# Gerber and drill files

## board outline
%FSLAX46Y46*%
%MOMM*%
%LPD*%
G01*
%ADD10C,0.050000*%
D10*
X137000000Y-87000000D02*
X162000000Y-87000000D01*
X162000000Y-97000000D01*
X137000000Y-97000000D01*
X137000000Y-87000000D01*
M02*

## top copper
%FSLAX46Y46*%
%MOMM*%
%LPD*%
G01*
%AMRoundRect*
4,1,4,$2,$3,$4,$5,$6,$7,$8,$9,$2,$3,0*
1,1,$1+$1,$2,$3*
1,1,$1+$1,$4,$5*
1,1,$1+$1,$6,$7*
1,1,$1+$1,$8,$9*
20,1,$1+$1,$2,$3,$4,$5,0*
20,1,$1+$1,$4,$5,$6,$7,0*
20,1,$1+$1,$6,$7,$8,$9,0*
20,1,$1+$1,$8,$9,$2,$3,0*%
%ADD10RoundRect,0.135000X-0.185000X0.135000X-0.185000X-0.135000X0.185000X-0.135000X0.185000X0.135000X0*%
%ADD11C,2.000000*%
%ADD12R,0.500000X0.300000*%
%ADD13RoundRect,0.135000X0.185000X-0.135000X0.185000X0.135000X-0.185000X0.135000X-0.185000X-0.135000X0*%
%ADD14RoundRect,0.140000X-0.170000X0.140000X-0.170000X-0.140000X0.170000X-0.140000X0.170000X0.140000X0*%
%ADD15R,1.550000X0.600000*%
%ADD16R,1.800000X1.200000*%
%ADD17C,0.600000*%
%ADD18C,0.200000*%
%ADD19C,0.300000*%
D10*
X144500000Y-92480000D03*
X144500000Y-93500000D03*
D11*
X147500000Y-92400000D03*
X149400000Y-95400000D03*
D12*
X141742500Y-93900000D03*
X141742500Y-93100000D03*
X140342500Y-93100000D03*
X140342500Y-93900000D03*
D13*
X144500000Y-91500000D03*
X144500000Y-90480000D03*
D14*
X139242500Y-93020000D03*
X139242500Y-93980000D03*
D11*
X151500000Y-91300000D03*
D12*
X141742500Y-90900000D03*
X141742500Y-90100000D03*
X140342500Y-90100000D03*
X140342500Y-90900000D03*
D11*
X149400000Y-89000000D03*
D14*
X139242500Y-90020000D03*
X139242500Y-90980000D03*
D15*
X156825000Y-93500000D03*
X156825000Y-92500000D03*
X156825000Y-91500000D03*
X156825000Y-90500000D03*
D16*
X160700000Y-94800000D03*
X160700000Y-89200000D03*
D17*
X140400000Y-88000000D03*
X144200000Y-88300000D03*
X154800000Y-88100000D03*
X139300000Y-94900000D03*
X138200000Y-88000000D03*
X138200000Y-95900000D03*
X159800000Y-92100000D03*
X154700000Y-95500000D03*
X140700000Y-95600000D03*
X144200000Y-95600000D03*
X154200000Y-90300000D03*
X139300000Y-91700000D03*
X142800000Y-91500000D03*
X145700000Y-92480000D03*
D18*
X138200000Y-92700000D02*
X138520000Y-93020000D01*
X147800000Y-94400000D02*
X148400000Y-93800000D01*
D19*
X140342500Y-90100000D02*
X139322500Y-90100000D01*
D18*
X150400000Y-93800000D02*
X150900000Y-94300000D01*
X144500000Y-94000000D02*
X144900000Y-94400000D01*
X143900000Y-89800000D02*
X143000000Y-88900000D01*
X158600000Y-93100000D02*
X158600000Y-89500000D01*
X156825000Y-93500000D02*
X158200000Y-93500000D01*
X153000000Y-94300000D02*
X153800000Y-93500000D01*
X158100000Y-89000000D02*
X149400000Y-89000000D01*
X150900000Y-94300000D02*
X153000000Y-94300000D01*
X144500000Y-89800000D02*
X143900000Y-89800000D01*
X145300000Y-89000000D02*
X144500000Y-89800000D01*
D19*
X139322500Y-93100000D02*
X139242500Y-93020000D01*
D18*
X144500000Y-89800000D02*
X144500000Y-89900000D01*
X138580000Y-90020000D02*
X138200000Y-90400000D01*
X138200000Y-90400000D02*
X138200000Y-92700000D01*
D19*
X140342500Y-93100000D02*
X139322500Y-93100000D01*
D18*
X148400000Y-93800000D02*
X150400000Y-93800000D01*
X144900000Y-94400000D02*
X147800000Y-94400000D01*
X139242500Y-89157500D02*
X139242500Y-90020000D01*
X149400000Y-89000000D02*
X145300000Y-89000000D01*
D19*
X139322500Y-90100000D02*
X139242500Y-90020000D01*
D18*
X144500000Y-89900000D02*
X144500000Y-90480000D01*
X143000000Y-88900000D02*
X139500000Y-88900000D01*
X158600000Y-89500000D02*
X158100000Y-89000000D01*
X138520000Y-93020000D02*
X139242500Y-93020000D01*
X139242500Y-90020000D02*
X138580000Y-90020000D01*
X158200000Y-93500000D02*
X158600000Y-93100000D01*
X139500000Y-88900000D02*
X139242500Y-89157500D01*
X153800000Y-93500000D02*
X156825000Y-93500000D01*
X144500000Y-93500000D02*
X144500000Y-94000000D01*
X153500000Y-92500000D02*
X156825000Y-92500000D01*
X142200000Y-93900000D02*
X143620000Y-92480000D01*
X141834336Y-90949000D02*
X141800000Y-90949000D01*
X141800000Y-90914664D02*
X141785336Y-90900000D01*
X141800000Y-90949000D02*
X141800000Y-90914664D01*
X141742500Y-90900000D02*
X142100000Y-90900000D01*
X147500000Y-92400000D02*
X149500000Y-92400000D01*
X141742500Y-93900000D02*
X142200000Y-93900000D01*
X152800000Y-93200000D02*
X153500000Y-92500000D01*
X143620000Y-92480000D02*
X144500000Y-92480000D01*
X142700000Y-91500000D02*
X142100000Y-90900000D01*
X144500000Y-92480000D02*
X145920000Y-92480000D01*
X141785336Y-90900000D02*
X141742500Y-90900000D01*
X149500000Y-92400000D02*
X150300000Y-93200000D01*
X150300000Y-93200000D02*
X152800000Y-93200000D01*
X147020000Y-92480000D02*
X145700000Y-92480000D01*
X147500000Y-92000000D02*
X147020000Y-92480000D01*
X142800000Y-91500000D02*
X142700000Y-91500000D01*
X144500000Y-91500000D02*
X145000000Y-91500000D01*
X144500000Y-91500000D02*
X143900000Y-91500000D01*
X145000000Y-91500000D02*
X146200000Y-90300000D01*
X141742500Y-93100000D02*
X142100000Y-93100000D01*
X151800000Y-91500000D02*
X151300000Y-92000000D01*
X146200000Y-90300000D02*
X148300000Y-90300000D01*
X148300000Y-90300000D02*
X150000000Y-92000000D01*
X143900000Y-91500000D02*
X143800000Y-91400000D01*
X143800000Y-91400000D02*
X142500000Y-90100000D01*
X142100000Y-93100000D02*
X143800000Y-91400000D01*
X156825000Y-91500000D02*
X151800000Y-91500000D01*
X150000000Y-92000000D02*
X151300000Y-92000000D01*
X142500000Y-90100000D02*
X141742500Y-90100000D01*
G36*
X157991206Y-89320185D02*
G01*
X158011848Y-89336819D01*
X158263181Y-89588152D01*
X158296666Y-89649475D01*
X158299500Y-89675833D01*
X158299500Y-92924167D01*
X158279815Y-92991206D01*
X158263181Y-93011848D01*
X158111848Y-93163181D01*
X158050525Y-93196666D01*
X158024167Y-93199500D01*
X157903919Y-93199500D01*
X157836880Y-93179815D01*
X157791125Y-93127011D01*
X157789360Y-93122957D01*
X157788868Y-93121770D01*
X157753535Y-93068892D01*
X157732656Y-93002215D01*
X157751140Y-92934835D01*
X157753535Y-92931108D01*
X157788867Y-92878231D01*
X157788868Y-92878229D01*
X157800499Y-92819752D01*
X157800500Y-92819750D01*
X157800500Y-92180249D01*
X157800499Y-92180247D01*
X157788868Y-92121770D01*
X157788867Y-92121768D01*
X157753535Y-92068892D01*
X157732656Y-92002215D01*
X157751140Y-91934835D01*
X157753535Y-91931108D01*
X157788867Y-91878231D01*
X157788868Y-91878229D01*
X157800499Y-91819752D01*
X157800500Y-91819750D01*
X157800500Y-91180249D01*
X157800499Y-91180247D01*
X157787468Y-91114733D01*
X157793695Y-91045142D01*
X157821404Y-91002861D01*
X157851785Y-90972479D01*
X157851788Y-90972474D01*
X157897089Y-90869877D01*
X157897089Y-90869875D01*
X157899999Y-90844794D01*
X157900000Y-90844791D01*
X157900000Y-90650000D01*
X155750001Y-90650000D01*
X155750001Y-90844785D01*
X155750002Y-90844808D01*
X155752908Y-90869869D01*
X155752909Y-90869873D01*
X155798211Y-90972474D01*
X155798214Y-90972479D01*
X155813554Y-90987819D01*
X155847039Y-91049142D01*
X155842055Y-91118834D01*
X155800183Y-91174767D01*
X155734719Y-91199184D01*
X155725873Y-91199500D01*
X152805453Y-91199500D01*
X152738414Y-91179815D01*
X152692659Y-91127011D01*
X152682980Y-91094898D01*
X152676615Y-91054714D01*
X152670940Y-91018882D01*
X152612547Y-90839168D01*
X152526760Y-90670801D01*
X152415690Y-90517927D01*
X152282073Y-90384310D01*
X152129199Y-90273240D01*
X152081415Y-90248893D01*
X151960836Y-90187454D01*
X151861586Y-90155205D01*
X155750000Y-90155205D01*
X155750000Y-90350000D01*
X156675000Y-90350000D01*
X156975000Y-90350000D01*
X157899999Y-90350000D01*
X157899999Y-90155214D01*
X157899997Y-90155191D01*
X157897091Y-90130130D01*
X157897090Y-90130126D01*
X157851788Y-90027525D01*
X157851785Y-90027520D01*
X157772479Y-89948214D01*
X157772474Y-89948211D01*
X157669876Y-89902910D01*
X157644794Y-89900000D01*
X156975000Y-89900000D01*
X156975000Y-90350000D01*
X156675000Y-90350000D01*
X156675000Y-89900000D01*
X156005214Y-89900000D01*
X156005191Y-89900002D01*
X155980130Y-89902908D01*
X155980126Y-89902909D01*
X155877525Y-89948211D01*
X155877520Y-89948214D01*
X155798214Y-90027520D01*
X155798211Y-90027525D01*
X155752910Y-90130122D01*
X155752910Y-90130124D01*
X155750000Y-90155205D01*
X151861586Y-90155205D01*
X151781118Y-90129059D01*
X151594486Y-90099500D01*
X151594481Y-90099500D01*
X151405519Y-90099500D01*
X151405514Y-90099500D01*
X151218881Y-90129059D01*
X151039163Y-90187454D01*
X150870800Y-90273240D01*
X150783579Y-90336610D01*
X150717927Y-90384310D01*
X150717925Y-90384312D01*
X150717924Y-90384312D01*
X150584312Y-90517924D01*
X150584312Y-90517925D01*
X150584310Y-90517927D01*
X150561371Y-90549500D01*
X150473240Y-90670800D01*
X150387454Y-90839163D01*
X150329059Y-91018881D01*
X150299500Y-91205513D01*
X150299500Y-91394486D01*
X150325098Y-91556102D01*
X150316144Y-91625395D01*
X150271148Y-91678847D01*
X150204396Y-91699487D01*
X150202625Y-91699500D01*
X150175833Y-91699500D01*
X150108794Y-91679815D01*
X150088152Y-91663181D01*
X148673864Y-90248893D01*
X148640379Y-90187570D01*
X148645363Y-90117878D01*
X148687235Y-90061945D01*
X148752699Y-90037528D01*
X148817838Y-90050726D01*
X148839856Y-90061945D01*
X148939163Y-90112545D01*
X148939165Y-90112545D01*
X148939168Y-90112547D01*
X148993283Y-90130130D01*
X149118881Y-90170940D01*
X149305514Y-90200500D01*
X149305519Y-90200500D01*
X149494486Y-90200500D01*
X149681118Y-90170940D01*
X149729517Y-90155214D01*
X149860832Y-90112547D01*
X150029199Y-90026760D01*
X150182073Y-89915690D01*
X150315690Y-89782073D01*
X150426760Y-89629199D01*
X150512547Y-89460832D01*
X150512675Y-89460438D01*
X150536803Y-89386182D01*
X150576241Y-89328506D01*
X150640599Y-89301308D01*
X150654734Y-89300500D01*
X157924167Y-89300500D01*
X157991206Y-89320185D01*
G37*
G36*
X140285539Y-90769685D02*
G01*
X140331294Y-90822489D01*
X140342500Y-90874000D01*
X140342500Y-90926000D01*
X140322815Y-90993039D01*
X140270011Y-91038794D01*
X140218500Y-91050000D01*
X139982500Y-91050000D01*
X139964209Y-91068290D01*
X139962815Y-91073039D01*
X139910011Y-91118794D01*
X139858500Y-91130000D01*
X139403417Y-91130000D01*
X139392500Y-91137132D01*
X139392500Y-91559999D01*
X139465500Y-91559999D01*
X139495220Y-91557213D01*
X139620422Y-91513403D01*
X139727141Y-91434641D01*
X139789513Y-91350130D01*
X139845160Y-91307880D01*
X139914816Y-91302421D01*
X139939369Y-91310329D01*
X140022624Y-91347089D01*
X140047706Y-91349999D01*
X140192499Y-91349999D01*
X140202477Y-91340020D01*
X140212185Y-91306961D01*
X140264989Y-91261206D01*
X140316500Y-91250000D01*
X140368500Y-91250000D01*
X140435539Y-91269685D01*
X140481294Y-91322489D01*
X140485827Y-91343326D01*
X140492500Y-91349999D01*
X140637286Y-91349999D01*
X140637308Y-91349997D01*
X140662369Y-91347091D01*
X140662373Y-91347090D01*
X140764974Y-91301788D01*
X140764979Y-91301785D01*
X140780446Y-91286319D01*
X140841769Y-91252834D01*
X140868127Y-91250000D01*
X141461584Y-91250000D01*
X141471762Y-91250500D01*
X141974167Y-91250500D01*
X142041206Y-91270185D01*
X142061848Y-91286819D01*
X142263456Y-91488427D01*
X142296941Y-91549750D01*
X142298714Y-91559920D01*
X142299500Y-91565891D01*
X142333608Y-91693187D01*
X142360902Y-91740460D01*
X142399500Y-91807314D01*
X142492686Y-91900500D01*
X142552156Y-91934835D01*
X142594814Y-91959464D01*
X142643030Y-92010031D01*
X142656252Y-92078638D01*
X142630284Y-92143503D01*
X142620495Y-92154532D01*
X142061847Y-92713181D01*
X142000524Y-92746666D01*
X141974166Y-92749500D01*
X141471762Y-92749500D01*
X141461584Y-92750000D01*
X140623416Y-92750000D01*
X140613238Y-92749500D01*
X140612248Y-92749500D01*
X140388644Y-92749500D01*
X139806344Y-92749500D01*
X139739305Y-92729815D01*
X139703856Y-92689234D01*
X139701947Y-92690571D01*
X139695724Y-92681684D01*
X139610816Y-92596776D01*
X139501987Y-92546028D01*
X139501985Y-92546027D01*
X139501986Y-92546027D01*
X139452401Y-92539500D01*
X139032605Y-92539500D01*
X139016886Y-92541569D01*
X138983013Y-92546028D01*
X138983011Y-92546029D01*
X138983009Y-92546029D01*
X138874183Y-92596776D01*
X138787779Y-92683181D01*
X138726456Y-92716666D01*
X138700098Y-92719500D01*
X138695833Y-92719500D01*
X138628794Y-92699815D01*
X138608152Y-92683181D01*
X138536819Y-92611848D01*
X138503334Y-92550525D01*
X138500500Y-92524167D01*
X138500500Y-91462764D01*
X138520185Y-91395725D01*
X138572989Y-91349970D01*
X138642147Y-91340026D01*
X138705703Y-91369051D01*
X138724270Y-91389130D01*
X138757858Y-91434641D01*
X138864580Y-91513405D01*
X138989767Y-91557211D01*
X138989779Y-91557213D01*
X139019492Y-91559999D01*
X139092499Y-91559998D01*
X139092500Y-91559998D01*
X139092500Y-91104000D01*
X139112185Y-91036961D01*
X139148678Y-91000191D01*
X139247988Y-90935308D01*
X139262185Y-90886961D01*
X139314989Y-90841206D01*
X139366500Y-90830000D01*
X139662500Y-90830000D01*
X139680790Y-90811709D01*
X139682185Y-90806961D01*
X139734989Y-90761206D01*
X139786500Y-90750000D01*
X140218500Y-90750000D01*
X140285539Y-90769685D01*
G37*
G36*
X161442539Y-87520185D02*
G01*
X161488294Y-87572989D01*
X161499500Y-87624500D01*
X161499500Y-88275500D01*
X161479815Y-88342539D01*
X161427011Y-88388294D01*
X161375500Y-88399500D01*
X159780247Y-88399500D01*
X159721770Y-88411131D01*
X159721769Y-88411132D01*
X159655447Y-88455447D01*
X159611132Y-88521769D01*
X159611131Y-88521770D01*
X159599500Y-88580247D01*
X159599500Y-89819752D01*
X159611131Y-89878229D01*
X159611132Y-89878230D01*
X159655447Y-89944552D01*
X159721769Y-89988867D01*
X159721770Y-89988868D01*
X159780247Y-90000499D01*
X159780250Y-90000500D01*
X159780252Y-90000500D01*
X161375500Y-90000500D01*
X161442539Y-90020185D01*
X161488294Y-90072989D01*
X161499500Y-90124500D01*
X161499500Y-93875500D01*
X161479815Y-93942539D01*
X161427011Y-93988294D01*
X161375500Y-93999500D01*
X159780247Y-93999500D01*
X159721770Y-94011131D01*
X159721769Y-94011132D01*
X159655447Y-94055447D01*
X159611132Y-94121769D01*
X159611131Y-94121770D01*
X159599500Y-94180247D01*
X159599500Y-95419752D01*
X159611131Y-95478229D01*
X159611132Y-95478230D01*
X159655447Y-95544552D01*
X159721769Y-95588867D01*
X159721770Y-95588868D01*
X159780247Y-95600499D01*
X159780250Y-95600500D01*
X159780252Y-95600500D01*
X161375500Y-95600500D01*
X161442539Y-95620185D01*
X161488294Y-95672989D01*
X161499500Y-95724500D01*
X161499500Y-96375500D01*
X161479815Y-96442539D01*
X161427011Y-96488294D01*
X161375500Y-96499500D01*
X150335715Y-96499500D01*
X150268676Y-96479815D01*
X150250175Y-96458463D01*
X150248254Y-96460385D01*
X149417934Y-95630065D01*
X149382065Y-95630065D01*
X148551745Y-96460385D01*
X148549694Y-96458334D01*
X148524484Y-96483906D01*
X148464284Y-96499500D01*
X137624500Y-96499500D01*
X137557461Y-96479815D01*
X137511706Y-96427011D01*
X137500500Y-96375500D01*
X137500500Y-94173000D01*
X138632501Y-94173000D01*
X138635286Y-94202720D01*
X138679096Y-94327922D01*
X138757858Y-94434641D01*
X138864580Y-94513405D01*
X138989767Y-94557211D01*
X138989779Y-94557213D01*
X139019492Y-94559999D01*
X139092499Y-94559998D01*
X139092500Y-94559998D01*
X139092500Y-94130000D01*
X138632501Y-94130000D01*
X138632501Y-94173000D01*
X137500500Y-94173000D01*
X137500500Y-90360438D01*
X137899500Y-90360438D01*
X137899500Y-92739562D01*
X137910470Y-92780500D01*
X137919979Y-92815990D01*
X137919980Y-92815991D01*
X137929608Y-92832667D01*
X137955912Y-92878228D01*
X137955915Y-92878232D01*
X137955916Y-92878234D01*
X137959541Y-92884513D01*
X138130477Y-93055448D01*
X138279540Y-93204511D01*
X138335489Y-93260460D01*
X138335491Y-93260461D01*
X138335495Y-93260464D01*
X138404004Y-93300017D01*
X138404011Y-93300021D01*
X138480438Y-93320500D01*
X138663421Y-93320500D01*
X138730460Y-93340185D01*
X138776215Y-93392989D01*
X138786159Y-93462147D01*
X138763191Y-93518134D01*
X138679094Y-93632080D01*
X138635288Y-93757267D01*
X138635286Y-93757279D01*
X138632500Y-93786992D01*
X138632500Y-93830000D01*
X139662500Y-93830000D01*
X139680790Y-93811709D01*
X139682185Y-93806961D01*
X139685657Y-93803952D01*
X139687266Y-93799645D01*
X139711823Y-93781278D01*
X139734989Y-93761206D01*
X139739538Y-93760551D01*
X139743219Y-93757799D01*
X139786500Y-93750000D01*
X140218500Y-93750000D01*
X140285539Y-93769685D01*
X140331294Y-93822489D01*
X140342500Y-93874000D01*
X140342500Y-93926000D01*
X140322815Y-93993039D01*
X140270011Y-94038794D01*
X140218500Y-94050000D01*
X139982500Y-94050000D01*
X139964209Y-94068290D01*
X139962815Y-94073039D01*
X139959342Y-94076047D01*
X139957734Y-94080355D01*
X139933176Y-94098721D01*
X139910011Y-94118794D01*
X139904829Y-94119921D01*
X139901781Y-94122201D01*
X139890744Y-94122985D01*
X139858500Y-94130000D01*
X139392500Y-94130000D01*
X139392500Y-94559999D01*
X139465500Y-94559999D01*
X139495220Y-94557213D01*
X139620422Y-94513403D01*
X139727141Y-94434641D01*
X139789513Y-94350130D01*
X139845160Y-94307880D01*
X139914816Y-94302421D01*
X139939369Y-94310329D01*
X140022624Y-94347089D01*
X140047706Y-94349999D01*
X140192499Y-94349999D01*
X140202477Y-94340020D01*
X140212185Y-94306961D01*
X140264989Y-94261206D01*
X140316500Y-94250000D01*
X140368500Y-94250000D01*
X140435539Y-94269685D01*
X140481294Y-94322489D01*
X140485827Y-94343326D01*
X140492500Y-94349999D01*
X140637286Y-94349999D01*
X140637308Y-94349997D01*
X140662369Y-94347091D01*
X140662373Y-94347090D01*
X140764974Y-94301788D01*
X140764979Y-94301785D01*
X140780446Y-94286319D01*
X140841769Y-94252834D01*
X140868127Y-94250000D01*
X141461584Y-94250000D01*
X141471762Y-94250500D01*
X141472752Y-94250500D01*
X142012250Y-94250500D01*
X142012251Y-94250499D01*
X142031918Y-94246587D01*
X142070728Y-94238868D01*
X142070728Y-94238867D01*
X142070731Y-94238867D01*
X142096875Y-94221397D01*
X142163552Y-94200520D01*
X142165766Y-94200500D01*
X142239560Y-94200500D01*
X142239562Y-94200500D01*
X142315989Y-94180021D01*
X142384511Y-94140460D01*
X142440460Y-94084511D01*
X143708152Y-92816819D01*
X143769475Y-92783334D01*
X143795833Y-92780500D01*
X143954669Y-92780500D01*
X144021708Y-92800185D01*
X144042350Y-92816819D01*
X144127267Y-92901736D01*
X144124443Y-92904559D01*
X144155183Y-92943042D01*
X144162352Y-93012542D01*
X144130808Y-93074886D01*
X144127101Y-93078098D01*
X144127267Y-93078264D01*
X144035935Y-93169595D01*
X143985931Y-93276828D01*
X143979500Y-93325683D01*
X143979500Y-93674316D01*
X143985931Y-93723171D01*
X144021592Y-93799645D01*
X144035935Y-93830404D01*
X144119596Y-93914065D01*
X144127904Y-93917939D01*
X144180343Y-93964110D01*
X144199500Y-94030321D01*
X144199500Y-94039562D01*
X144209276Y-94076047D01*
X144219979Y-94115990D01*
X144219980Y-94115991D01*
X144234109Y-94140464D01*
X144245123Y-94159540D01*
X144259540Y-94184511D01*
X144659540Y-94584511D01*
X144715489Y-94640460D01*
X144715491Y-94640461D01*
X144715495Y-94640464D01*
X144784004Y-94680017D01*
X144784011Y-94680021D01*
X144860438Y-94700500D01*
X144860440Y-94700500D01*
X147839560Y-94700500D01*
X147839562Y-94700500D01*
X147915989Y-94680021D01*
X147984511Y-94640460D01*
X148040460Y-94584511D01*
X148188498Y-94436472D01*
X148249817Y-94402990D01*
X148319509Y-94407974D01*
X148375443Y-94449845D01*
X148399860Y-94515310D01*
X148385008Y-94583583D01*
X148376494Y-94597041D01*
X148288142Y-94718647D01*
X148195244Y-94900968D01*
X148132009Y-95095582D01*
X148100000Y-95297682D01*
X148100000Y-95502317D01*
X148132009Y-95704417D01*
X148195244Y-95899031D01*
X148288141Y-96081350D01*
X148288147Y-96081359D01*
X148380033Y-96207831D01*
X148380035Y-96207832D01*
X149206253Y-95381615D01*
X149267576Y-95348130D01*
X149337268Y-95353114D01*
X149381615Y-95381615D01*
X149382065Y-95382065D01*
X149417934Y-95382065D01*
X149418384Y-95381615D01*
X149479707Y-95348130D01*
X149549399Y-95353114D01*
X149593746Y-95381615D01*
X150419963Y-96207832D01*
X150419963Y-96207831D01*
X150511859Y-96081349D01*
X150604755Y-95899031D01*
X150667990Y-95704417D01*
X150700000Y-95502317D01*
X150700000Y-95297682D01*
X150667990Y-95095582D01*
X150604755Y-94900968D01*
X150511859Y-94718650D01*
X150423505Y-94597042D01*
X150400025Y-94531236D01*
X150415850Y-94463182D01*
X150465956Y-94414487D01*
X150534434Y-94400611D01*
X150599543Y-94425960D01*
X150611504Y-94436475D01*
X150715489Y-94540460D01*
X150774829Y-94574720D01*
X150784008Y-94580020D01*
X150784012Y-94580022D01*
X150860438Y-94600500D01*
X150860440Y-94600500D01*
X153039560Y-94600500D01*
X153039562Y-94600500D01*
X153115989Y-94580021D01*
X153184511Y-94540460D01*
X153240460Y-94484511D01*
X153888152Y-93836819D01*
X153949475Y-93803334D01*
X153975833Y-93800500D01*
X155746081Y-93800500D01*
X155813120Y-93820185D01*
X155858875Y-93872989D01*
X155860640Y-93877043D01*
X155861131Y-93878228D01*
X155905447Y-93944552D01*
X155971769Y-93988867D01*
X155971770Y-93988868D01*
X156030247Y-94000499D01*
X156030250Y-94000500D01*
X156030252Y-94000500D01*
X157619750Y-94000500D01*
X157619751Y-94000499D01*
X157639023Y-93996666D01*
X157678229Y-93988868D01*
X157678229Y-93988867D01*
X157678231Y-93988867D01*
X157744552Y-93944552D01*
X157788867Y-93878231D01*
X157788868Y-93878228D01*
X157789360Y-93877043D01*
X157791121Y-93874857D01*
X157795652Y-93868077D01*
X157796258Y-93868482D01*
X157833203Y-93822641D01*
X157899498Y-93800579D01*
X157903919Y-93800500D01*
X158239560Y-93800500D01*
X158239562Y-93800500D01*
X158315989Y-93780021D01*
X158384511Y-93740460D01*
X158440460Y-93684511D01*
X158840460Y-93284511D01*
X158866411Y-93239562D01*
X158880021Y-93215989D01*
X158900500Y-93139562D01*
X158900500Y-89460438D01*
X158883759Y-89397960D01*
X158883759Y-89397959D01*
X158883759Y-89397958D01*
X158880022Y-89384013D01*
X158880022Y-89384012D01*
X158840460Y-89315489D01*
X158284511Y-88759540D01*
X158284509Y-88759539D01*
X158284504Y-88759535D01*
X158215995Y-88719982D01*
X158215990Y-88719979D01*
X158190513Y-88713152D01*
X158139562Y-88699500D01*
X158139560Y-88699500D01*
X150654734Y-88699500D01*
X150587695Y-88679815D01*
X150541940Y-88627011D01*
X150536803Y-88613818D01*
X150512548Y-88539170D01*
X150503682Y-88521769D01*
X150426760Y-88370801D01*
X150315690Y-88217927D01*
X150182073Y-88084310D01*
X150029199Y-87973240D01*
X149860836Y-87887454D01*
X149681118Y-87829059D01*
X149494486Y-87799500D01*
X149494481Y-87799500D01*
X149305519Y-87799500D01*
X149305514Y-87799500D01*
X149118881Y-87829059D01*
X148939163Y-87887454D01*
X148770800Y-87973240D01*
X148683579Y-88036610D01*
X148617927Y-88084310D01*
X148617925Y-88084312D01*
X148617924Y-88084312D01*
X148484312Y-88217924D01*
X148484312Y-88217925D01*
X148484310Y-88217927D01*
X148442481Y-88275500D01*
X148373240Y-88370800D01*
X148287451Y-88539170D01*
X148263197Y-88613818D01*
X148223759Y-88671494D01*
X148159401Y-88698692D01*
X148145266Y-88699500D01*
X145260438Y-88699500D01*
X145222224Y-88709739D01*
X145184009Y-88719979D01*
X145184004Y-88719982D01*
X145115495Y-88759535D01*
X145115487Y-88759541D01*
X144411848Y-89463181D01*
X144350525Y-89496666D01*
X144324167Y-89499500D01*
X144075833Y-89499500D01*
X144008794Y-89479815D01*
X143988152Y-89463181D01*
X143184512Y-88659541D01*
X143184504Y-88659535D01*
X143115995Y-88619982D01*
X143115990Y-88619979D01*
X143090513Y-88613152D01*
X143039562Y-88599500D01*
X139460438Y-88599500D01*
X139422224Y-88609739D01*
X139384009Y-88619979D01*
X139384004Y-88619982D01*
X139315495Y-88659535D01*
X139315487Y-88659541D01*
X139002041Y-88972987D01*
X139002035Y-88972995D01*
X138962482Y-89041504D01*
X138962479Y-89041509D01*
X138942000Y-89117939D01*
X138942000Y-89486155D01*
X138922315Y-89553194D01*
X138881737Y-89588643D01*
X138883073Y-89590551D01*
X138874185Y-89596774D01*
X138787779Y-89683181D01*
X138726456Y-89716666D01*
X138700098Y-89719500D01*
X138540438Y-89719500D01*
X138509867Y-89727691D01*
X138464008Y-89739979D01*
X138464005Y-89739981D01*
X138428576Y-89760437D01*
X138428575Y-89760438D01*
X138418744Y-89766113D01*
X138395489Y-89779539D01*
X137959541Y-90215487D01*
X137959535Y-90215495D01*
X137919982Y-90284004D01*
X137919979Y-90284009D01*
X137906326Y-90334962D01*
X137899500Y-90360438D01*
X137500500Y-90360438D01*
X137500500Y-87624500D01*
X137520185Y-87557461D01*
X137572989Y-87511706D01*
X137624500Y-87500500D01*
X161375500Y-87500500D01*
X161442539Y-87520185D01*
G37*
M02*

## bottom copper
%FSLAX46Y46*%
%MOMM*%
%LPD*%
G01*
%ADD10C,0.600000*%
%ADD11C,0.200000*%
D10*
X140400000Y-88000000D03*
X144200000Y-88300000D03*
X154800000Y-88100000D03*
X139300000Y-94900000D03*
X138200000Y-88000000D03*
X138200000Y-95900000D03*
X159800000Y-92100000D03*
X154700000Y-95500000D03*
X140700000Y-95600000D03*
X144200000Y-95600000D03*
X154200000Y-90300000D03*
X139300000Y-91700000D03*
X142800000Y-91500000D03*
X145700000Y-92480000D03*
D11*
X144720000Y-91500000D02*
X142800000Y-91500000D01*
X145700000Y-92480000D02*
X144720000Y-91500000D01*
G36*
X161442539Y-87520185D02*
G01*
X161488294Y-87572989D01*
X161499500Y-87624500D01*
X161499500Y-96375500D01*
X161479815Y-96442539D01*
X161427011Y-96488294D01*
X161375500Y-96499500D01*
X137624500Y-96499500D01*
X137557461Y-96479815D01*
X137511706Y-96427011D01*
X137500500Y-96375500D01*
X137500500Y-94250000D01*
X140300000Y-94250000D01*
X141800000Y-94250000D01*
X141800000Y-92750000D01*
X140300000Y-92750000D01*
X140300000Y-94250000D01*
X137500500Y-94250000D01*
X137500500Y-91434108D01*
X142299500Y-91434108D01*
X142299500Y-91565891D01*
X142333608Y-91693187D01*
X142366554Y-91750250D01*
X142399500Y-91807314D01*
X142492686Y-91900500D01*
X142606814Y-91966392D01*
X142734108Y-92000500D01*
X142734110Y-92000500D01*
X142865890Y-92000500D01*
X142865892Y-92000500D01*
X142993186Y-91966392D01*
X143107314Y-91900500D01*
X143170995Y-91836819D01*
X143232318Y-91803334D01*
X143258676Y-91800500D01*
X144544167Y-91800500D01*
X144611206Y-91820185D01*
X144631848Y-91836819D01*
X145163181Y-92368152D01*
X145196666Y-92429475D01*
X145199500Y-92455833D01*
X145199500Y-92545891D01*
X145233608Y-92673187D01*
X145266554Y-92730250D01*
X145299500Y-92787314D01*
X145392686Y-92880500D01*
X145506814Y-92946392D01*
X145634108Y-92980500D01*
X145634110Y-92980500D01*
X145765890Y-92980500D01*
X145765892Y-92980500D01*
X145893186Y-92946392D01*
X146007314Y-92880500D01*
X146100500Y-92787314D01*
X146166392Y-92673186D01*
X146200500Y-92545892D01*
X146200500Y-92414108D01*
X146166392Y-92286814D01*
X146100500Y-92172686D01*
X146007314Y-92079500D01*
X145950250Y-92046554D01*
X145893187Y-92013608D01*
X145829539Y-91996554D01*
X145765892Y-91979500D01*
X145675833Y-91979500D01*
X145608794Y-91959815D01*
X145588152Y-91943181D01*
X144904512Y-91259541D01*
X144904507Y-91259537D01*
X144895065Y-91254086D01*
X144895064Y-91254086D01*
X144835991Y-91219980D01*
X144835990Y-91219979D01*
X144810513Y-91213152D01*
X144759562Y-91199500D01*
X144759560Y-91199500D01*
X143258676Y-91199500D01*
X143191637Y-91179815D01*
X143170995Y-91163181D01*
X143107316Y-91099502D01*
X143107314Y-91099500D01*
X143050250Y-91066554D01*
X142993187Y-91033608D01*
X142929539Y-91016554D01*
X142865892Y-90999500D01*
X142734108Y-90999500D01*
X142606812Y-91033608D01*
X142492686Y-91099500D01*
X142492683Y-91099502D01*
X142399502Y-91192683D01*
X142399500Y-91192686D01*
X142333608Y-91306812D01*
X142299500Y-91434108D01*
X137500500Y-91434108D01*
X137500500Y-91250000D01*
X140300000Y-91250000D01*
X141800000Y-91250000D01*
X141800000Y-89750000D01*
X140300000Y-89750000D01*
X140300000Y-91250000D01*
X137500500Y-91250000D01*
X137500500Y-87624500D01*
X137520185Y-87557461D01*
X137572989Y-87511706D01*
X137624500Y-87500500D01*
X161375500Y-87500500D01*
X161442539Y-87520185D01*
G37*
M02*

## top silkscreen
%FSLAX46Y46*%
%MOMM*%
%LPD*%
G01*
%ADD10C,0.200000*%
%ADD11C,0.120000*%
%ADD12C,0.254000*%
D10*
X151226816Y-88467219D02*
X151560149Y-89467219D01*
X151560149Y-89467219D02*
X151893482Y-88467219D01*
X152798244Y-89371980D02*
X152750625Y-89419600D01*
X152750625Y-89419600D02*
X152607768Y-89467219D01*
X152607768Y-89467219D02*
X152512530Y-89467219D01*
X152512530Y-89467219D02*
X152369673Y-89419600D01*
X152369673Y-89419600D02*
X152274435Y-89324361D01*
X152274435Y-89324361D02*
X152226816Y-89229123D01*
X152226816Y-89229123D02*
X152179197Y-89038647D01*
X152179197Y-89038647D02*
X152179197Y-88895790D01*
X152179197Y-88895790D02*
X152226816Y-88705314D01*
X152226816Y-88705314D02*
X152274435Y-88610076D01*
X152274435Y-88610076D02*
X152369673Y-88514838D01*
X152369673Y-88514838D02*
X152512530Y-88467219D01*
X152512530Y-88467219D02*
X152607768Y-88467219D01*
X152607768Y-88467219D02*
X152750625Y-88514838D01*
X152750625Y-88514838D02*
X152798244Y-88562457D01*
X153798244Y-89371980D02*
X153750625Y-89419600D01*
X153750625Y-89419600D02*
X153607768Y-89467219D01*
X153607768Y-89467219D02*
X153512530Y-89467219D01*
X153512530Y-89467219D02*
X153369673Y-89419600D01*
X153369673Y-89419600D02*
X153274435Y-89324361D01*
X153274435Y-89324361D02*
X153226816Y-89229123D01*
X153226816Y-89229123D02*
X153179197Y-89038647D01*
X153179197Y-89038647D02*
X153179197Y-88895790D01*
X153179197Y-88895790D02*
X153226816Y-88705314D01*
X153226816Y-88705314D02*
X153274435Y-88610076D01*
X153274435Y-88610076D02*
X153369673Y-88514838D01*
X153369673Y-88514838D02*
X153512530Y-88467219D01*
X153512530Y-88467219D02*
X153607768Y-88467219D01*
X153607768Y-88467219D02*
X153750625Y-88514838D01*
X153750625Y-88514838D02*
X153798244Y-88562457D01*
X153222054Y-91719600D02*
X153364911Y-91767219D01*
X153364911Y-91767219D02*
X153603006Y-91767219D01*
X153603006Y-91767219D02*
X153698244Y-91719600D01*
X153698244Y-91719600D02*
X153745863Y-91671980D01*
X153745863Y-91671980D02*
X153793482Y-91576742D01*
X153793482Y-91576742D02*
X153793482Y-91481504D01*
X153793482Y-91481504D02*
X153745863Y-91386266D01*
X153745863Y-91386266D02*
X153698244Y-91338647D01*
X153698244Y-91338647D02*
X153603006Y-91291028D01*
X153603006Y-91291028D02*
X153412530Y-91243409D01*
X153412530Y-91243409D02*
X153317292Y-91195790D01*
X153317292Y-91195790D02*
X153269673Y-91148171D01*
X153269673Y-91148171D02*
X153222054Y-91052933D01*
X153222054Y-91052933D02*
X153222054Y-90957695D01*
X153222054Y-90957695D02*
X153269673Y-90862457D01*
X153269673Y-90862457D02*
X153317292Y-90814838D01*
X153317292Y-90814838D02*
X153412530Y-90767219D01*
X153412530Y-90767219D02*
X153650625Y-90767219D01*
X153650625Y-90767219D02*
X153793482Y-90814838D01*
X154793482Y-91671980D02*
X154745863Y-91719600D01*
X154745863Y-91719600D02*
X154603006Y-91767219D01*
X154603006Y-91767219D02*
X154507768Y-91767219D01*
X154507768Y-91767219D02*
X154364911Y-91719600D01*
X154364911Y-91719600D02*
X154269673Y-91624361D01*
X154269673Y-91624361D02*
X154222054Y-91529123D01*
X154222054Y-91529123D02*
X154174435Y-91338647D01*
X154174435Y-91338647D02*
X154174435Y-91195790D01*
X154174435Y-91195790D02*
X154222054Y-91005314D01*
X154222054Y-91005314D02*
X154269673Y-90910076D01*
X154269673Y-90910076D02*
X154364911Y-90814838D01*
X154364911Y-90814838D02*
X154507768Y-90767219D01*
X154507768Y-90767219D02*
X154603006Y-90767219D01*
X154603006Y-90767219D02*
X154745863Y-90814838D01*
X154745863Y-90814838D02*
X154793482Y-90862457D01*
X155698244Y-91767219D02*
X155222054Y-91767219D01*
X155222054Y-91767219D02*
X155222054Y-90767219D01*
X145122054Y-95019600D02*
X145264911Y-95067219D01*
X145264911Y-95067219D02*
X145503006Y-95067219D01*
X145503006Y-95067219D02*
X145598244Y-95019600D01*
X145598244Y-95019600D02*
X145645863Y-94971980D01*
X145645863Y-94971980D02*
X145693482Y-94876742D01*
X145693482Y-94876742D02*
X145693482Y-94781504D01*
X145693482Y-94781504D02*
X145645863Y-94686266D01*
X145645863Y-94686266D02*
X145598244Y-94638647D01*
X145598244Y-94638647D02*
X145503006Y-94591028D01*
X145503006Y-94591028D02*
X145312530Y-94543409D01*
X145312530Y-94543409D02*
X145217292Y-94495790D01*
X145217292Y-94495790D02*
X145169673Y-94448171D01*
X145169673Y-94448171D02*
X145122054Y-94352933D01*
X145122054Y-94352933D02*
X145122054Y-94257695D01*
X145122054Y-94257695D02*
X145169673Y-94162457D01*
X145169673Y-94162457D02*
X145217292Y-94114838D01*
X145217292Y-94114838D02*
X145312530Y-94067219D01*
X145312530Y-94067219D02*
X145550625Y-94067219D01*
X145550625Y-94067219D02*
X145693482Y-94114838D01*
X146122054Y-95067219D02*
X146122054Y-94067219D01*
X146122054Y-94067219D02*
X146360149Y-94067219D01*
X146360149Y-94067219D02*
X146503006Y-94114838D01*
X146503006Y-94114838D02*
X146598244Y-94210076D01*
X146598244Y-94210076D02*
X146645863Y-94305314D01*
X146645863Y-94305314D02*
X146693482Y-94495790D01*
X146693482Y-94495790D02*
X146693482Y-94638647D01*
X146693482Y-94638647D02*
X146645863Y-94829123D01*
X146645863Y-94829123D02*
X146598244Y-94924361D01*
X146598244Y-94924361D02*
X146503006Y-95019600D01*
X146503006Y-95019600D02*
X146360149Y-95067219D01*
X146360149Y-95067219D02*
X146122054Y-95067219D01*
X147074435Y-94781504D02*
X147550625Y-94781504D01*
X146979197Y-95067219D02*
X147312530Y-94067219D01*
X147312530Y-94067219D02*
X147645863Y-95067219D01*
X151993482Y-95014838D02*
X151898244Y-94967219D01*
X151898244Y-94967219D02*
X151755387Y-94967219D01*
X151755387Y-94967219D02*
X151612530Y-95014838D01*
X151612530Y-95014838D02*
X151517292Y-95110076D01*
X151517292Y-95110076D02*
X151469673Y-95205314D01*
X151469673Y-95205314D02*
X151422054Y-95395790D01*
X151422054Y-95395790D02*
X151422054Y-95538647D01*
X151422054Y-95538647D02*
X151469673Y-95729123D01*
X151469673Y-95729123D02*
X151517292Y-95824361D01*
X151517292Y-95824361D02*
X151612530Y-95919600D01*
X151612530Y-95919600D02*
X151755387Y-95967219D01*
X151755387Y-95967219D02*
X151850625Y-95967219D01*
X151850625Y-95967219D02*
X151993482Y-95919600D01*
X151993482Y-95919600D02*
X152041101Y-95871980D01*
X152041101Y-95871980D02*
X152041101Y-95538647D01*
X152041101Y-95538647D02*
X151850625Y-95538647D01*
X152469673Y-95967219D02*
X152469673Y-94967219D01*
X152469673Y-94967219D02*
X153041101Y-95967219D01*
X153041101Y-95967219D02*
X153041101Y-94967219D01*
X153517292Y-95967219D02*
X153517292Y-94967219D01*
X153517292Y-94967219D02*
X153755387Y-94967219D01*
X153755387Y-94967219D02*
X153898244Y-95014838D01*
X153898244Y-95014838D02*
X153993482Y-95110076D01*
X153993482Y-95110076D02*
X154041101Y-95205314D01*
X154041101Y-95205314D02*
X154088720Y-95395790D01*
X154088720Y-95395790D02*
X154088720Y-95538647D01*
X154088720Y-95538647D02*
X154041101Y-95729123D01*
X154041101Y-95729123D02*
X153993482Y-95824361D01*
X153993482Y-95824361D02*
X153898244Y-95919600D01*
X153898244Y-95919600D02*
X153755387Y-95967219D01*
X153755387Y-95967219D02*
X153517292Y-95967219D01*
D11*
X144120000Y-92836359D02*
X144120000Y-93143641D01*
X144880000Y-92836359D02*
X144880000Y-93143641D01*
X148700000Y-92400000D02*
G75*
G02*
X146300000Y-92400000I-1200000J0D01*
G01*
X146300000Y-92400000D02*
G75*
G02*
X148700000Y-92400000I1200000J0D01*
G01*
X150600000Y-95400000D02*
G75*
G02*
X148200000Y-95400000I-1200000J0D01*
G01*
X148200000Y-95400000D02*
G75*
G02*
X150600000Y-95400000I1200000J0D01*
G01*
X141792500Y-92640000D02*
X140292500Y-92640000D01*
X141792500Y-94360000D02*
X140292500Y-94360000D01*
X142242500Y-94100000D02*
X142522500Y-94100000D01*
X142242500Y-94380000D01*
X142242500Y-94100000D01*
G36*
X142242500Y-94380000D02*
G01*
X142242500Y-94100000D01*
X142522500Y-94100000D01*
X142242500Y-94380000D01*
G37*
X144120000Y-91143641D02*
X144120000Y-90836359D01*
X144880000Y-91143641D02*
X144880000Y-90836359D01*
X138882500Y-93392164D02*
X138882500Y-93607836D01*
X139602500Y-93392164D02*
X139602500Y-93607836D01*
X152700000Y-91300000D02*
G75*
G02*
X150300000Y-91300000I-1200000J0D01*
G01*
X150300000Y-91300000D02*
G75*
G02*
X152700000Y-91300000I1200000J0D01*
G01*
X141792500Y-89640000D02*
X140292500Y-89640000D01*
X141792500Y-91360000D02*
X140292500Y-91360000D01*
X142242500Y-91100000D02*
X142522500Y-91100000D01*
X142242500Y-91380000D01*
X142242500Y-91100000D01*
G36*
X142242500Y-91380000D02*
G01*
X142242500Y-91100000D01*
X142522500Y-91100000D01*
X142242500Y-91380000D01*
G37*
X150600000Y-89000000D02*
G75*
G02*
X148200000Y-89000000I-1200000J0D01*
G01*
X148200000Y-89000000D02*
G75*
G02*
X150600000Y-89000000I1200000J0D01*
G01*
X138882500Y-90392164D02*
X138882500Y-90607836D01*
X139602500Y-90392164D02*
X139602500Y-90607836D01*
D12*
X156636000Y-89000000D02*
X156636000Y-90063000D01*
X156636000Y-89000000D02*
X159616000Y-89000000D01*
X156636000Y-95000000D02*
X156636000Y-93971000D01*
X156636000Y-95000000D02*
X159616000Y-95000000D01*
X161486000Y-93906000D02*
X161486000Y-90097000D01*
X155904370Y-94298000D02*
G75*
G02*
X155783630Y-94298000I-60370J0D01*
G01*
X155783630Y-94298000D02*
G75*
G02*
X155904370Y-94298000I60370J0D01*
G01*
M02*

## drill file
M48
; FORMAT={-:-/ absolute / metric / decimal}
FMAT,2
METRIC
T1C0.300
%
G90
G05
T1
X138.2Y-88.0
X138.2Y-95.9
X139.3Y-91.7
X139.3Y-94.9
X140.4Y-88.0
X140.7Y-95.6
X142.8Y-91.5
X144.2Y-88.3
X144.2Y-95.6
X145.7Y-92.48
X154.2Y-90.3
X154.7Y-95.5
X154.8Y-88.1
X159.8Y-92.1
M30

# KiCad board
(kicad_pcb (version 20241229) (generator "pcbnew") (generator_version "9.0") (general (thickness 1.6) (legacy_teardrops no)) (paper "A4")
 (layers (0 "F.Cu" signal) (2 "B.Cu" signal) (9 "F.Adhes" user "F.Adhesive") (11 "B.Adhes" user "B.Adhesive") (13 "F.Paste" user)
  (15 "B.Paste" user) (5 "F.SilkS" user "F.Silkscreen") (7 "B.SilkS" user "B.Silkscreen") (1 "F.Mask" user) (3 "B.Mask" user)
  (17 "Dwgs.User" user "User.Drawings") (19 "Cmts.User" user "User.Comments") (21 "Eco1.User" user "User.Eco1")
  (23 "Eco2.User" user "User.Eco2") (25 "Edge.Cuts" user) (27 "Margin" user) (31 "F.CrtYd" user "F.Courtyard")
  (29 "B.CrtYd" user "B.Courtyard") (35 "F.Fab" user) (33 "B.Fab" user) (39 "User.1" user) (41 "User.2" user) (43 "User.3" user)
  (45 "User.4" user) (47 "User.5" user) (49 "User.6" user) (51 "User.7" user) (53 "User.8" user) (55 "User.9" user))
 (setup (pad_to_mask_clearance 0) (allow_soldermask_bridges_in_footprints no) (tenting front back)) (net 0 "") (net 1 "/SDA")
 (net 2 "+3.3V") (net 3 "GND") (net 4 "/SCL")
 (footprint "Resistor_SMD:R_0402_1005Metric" (layer "F.Cu") (at 144.5 92.99 -90)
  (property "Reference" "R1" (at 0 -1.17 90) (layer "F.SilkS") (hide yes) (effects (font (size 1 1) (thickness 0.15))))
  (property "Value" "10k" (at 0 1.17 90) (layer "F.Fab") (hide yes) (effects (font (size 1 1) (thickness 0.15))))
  (fp_line (start -0.153641 0.38) (end 0.153641 0.38) (stroke (width 0.12) (type solid)) (layer "F.SilkS"))
  (fp_line (start -0.153641 -0.38) (end 0.153641 -0.38) (stroke (width 0.12) (type solid)) (layer "F.SilkS"))
  (pad "1" smd roundrect (at -0.51 0 270) (size 0.54 0.64) (layers "F.Cu" "F.Mask" "F.Paste") (roundrect_rratio 0.25) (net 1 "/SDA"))
  (pad "2" smd roundrect (at 0.51 0 270) (size 0.54 0.64) (layers "F.Cu" "F.Mask" "F.Paste") (roundrect_rratio 0.25) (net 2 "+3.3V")))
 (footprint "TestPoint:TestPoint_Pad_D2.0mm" (layer "F.Cu") (at 147.5 92.4)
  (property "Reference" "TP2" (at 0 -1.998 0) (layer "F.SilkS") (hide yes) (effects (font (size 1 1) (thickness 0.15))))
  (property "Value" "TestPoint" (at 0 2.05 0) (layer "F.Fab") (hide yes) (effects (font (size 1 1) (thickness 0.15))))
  (fp_circle (center 0 0) (end 0 1.2) (stroke (width 0.12) (type solid)) (fill no) (layer "F.SilkS"))
  (pad "1" smd circle (at 0 0) (size 2 2) (layers "F.Cu" "F.Mask") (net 1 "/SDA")))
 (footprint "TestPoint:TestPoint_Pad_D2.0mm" (layer "F.Cu") (at 149.4 95.4)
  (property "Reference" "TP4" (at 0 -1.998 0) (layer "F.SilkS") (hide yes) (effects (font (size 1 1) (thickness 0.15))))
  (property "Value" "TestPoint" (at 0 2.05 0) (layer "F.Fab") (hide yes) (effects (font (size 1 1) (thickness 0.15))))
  (fp_circle (center 0 0) (end 0 1.2) (stroke (width 0.12) (type solid)) (fill no) (layer "F.SilkS"))
  (pad "1" smd circle (at 0 0) (size 2 2) (layers "F.Cu" "F.Mask") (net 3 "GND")))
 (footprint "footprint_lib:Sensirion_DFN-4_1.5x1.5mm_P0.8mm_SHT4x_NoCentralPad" (layer "F.Cu") (at 141.0425 93.5 180)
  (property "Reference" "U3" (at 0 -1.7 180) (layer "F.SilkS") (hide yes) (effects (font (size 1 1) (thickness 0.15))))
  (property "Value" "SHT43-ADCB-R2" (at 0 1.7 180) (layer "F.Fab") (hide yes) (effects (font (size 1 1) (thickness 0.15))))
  (fp_line (start -0.75 0.86) (end 0.75 0.86) (stroke (width 0.12) (type solid)) (layer "F.SilkS"))
  (fp_line (start -0.75 -0.86) (end 0.75 -0.86) (stroke (width 0.12) (type solid)) (layer "F.SilkS"))
  (fp_poly
   (pts (xy -1.2 -0.6) (xy -1.48 -0.6) (xy -1.2 -0.88) (xy -1.2 -0.6)) (stroke (width 0.12) (type solid)) (fill yes) (layer "F.SilkS"))
  (pad "1" smd rect (at -0.7 -0.4 180) (size 0.5 0.3) (layers "F.Cu" "F.Mask" "F.Paste") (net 1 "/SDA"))
  (pad "2" smd rect (at -0.7 0.4 180) (size 0.5 0.3) (layers "F.Cu" "F.Mask" "F.Paste") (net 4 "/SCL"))
  (pad "3" smd rect (at 0.7 0.4 180) (size 0.5 0.3) (layers "F.Cu" "F.Mask" "F.Paste") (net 2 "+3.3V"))
  (pad "4" smd rect (at 0.7 -0.4 180) (size 0.5 0.3) (layers "F.Cu" "F.Mask" "F.Paste") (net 3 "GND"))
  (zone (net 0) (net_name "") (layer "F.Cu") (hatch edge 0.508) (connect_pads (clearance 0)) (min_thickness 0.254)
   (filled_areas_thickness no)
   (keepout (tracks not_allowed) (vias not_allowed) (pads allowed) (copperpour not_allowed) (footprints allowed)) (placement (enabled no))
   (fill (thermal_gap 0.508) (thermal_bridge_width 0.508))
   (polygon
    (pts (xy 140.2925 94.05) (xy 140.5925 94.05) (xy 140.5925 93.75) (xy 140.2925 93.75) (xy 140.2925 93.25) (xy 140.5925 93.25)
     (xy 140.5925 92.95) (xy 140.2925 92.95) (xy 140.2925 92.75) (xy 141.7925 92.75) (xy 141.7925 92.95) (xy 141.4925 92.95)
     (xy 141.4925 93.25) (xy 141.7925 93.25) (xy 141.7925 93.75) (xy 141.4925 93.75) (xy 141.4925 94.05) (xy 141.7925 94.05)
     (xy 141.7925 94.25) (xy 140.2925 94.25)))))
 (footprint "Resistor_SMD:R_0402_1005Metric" (layer "F.Cu") (at 144.5 90.99 90)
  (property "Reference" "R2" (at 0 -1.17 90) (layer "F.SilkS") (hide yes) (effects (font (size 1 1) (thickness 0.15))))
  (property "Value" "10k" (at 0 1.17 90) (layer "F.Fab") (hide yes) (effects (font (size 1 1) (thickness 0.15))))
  (fp_line (start -0.153641 -0.38) (end 0.153641 -0.38) (stroke (width 0.12) (type solid)) (layer "F.SilkS"))
  (fp_line (start -0.153641 0.38) (end 0.153641 0.38) (stroke (width 0.12) (type solid)) (layer "F.SilkS"))
  (pad "1" smd roundrect (at -0.51 0 90) (size 0.54 0.64) (layers "F.Cu" "F.Mask" "F.Paste") (roundrect_rratio 0.25) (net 4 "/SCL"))
  (pad "2" smd roundrect (at 0.51 0 90) (size 0.54 0.64) (layers "F.Cu" "F.Mask" "F.Paste") (roundrect_rratio 0.25) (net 2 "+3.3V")))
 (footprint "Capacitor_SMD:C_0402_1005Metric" (layer "F.Cu") (at 139.2425 93.5 -90)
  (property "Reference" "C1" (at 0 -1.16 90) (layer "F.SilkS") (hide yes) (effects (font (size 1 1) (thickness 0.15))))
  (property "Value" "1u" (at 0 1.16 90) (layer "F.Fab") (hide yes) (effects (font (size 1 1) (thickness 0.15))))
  (fp_line (start -0.107836 0.36) (end 0.107836 0.36) (stroke (width 0.12) (type solid)) (layer "F.SilkS"))
  (fp_line (start -0.107836 -0.36) (end 0.107836 -0.36) (stroke (width 0.12) (type solid)) (layer "F.SilkS"))
  (pad "1" smd roundrect (at -0.48 0 270) (size 0.56 0.62) (layers "F.Cu" "F.Mask" "F.Paste") (roundrect_rratio 0.25) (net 2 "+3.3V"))
  (pad "2" smd roundrect (at 0.48 0 270) (size 0.56 0.62) (layers "F.Cu" "F.Mask" "F.Paste") (roundrect_rratio 0.25) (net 3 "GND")))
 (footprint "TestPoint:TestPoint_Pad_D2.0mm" (layer "F.Cu") (at 151.5 91.3)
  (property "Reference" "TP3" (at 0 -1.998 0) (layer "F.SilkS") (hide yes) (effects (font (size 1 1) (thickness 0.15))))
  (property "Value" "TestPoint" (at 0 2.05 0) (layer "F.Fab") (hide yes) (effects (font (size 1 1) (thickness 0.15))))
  (fp_circle (center 0 0) (end 0 1.2) (stroke (width 0.12) (type solid)) (fill no) (layer "F.SilkS"))
  (pad "1" smd circle (at 0 0) (size 2 2) (layers "F.Cu" "F.Mask") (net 4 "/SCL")))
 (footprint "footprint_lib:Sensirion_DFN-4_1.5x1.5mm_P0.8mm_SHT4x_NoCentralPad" (layer "F.Cu") (at 141.0425 90.5 180)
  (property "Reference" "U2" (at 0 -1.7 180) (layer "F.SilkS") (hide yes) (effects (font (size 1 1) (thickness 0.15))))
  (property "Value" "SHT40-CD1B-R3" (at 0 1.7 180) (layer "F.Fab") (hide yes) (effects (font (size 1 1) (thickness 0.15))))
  (fp_line (start -0.75 0.86) (end 0.75 0.86) (stroke (width 0.12) (type solid)) (layer "F.SilkS"))
  (fp_line (start -0.75 -0.86) (end 0.75 -0.86) (stroke (width 0.12) (type solid)) (layer "F.SilkS"))
  (fp_poly
   (pts (xy -1.2 -0.6) (xy -1.48 -0.6) (xy -1.2 -0.88) (xy -1.2 -0.6)) (stroke (width 0.12) (type solid)) (fill yes) (layer "F.SilkS"))
  (pad "1" smd rect (at -0.7 -0.4 180) (size 0.5 0.3) (layers "F.Cu" "F.Mask" "F.Paste") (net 1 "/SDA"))
  (pad "2" smd rect (at -0.7 0.4 180) (size 0.5 0.3) (layers "F.Cu" "F.Mask" "F.Paste") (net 4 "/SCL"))
  (pad "3" smd rect (at 0.7 0.4 180) (size 0.5 0.3) (layers "F.Cu" "F.Mask" "F.Paste") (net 2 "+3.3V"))
  (pad "4" smd rect (at 0.7 -0.4 180) (size 0.5 0.3) (layers "F.Cu" "F.Mask" "F.Paste") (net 3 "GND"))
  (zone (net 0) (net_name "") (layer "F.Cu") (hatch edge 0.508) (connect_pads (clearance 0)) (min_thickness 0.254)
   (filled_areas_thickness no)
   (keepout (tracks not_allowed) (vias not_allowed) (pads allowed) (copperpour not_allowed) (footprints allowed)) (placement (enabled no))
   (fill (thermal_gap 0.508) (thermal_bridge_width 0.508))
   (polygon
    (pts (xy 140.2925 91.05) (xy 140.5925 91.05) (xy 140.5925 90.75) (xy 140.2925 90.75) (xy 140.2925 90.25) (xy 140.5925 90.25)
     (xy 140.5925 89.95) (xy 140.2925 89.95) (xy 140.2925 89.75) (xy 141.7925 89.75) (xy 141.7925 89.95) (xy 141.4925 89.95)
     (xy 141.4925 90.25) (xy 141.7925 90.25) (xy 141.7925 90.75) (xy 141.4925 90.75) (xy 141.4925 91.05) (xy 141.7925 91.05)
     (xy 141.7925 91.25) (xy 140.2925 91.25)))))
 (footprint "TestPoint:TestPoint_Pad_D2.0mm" (layer "F.Cu") (at 149.4 89)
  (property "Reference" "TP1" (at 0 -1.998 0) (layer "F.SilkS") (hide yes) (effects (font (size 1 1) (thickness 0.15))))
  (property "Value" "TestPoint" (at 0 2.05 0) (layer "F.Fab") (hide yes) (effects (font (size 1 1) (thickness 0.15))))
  (fp_circle (center 0 0) (end 0 1.2) (stroke (width 0.12) (type solid)) (fill no) (layer "F.SilkS"))
  (pad "1" smd circle (at 0 0) (size 2 2) (layers "F.Cu" "F.Mask") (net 2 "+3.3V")))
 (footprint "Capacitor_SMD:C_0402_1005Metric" (layer "F.Cu") (at 139.2425 90.5 -90)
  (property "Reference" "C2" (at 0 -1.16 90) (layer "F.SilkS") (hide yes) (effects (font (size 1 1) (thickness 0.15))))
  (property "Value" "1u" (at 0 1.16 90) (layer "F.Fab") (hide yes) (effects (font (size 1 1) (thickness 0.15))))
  (fp_line (start -0.107836 0.36) (end 0.107836 0.36) (stroke (width 0.12) (type solid)) (layer "F.SilkS"))
  (fp_line (start -0.107836 -0.36) (end 0.107836 -0.36) (stroke (width 0.12) (type solid)) (layer "F.SilkS"))
  (pad "1" smd roundrect (at -0.48 0 270) (size 0.56 0.62) (layers "F.Cu" "F.Mask" "F.Paste") (roundrect_rratio 0.25) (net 2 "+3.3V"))
  (pad "2" smd roundrect (at 0.48 0 270) (size 0.56 0.62) (layers "F.Cu" "F.Mask" "F.Paste") (roundrect_rratio 0.25) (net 3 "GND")))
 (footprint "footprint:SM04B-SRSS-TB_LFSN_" (layer "F.Cu") (at 161.486 95 90)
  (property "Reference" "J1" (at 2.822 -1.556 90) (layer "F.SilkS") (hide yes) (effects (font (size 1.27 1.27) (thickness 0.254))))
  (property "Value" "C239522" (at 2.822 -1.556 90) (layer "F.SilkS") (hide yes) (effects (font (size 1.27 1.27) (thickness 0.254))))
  (fp_line (start 6 -4.85) (end 4.937 -4.85) (stroke (width 0.254) (type solid)) (layer "F.SilkS"))
  (fp_line (start 6 -4.85) (end 6 -1.87) (stroke (width 0.254) (type solid)) (layer "F.SilkS"))
  (fp_line (start 0 -4.85) (end 1.029 -4.85) (stroke (width 0.254) (type solid)) (layer "F.SilkS"))
  (fp_line (start 0 -4.85) (end 0 -1.87) (stroke (width 0.254) (type solid)) (layer "F.SilkS"))
  (fp_line (start 1.094 0) (end 4.903 0) (stroke (width 0.254) (type solid)) (layer "F.SilkS"))
  (fp_circle (center 0.702 -5.642) (end 0.702 -5.58163) (stroke (width 0.254) (type solid)) (fill no) (layer "F.SilkS"))
  (pad "1" smd rect (at 1.5 -4.661 90) (size 0.6 1.55) (layers "F.Cu" "F.Mask" "F.Paste") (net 2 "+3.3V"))
  (pad "2" smd rect (at 2.5 -4.661 90) (size 0.6 1.55) (layers "F.Cu" "F.Mask" "F.Paste") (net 1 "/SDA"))
  (pad "3" smd rect (at 3.5 -4.661 90) (size 0.6 1.55) (layers "F.Cu" "F.Mask" "F.Paste") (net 4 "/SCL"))
  (pad "4" smd rect (at 4.5 -4.661 90) (size 0.6 1.55) (layers "F.Cu" "F.Mask" "F.Paste") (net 3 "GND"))
  (pad "5" smd rect (at 0.2 -0.786 90) (size 1.2 1.8) (layers "F.Cu" "F.Mask" "F.Paste"))
  (pad "6" smd rect (at 5.8 -0.786 90) (size 1.2 1.8) (layers "F.Cu" "F.Mask" "F.Paste")))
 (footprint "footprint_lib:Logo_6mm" (layer "B.Cu") (at 152.2 91.8 180)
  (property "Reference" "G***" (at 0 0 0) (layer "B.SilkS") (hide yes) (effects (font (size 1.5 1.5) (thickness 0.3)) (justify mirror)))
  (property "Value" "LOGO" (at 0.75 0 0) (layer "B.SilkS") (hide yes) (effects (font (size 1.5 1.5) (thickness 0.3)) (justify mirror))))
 (gr_rect (start 137 87) (end 162 97) (stroke (width 0.05) (type default)) (fill no) (layer "Edge.Cuts"))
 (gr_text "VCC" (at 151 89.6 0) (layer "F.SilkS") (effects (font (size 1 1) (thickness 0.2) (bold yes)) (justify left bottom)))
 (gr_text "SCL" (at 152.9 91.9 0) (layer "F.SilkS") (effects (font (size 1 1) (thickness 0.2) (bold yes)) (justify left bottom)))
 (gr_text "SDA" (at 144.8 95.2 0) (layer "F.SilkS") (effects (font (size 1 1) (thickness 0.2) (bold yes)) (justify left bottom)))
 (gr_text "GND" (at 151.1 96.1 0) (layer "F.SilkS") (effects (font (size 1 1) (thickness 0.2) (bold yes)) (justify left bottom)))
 (segment (start 138.2 92.7) (end 138.52 93.02) (width 0.2) (layer "F.Cu") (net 2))
 (segment (start 147.8 94.4) (end 148.4 93.8) (width 0.2) (layer "F.Cu") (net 2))
 (segment (start 140.3425 90.1) (end 139.3225 90.1) (width 0.3) (layer "F.Cu") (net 2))
 (segment (start 150.4 93.8) (end 150.9 94.3) (width 0.2) (layer "F.Cu") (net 2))
 (segment (start 144.5 94) (end 144.9 94.4) (width 0.2) (layer "F.Cu") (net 2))
 (segment (start 143.9 89.8) (end 143 88.9) (width 0.2) (layer "F.Cu") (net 2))
 (segment (start 158.6 93.1) (end 158.6 89.5) (width 0.2) (layer "F.Cu") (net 2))
 (segment (start 156.825 93.5) (end 158.2 93.5) (width 0.2) (layer "F.Cu") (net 2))
 (segment (start 153 94.3) (end 153.8 93.5) (width 0.2) (layer "F.Cu") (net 2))
 (segment (start 158.1 89) (end 149.4 89) (width 0.2) (layer "F.Cu") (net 2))
 (segment (start 150.9 94.3) (end 153 94.3) (width 0.2) (layer "F.Cu") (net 2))
 (segment (start 144.5 89.8) (end 143.9 89.8) (width 0.2) (layer "F.Cu") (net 2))
 (segment (start 145.3 89) (end 144.5 89.8) (width 0.2) (layer "F.Cu") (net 2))
 (segment (start 139.3225 93.1) (end 139.2425 93.02) (width 0.3) (layer "F.Cu") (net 2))
 (segment (start 144.5 89.8) (end 144.5 89.9) (width 0.2) (layer "F.Cu") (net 2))
 (segment (start 138.58 90.02) (end 138.2 90.4) (width 0.2) (layer "F.Cu") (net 2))
 (segment (start 138.2 90.4) (end 138.2 92.7) (width 0.2) (layer "F.Cu") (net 2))
 (segment (start 140.3425 93.1) (end 139.3225 93.1) (width 0.3) (layer "F.Cu") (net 2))
 (segment (start 148.4 93.8) (end 150.4 93.8) (width 0.2) (layer "F.Cu") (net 2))
 (segment (start 144.9 94.4) (end 147.8 94.4) (width 0.2) (layer "F.Cu") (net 2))
 (segment (start 139.2425 89.1575) (end 139.2425 90.02) (width 0.2) (layer "F.Cu") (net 2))
 (segment (start 149.4 89) (end 145.3 89) (width 0.2) (layer "F.Cu") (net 2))
 (segment (start 139.3225 90.1) (end 139.2425 90.02) (width 0.3) (layer "F.Cu") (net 2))
 (segment (start 144.5 89.9) (end 144.5 90.48) (width 0.2) (layer "F.Cu") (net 2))
 (segment (start 143 88.9) (end 139.5 88.9) (width 0.2) (layer "F.Cu") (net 2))
 (segment (start 158.6 89.5) (end 158.1 89) (width 0.2) (layer "F.Cu") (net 2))
 (segment (start 138.52 93.02) (end 139.2425 93.02) (width 0.2) (layer "F.Cu") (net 2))
 (segment (start 139.2425 90.02) (end 138.58 90.02) (width 0.2) (layer "F.Cu") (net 2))
 (segment (start 158.2 93.5) (end 158.6 93.1) (width 0.2) (layer "F.Cu") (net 2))
 (segment (start 139.5 88.9) (end 139.2425 89.1575) (width 0.2) (layer "F.Cu") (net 2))
 (segment (start 153.8 93.5) (end 156.825 93.5) (width 0.2) (layer "F.Cu") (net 2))
 (segment (start 144.5 93.5) (end 144.5 94) (width 0.2) (layer "F.Cu") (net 2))
 (via (at 140.4 88) (size 0.6) (drill 0.3) (layers "F.Cu" "B.Cu") (free yes) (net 3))
 (via (at 144.2 88.3) (size 0.6) (drill 0.3) (layers "F.Cu" "B.Cu") (free yes) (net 3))
 (via (at 154.8 88.1) (size 0.6) (drill 0.3) (layers "F.Cu" "B.Cu") (free yes) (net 3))
 (via (at 139.3 94.9) (size 0.6) (drill 0.3) (layers "F.Cu" "B.Cu") (free yes) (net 3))
 (via (at 138.2 88) (size 0.6) (drill 0.3) (layers "F.Cu" "B.Cu") (free yes) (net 3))
 (via (at 138.2 95.9) (size 0.6) (drill 0.3) (layers "F.Cu" "B.Cu") (free yes) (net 3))
 (via (at 159.8 92.1) (size 0.6) (drill 0.3) (layers "F.Cu" "B.Cu") (free yes) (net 3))
 (via (at 154.7 95.5) (size 0.6) (drill 0.3) (layers "F.Cu" "B.Cu") (free yes) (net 3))
 (via (at 140.7 95.6) (size 0.6) (drill 0.3) (layers "F.Cu" "B.Cu") (free yes) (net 3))
 (via (at 144.2 95.6) (size 0.6) (drill 0.3) (layers "F.Cu" "B.Cu") (free yes) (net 3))
 (via (at 154.2 90.3) (size 0.6) (drill 0.3) (layers "F.Cu" "B.Cu") (free yes) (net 3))
 (via (at 139.3 91.7) (size 0.6) (drill 0.3) (layers "F.Cu" "B.Cu") (free yes) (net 3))
 (segment (start 153.5 92.5) (end 156.825 92.5) (width 0.2) (layer "F.Cu") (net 1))
 (segment (start 142.2 93.9) (end 143.62 92.48) (width 0.2) (layer "F.Cu") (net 1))
 (segment (start 141.834336 90.949) (end 141.8 90.949) (width 0.2) (layer "F.Cu") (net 1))
 (segment (start 141.8 90.914664) (end 141.785336 90.9) (width 0.2) (layer "F.Cu") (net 1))
 (segment (start 141.8 90.949) (end 141.8 90.914664) (width 0.2) (layer "F.Cu") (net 1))
 (segment (start 141.7425 90.9) (end 142.1 90.9) (width 0.2) (layer "F.Cu") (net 1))
 (segment (start 147.5 92.4) (end 149.5 92.4) (width 0.2) (layer "F.Cu") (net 1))
 (segment (start 141.7425 93.9) (end 142.2 93.9) (width 0.2) (layer "F.Cu") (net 1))
 (segment (start 152.8 93.2) (end 153.5 92.5) (width 0.2) (layer "F.Cu") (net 1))
 (segment (start 143.62 92.48) (end 144.5 92.48) (width 0.2) (layer "F.Cu") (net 1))
 (segment (start 142.7 91.5) (end 142.1 90.9) (width 0.2) (layer "F.Cu") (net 1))
 (segment (start 144.5 92.48) (end 145.92 92.48) (width 0.2) (layer "F.Cu") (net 1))
 (segment (start 141.785336 90.9) (end 141.7425 90.9) (width 0.2) (layer "F.Cu") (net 1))
 (segment (start 149.5 92.4) (end 150.3 93.2) (width 0.2) (layer "F.Cu") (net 1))
 (segment (start 150.3 93.2) (end 152.8 93.2) (width 0.2) (layer "F.Cu") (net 1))
 (segment (start 147.02 92.48) (end 145.7 92.48) (width 0.2) (layer "F.Cu") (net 1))
 (segment (start 147.5 92) (end 147.02 92.48) (width 0.2) (layer "F.Cu") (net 1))
 (segment (start 142.8 91.5) (end 142.7 91.5) (width 0.2) (layer "F.Cu") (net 1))
 (via (at 142.8 91.5) (size 0.6) (drill 0.3) (layers "F.Cu" "B.Cu") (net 1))
 (via (at 145.7 92.48) (size 0.6) (drill 0.3) (layers "F.Cu" "B.Cu") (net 1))
 (segment (start 144.72 91.5) (end 142.8 91.5) (width 0.2) (layer "B.Cu") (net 1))
 (segment (start 145.7 92.48) (end 144.72 91.5) (width 0.2) (layer "B.Cu") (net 1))
 (segment (start 144.5 91.5) (end 145 91.5) (width 0.2) (layer "F.Cu") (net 4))
 (segment (start 144.5 91.5) (end 143.9 91.5) (width 0.2) (layer "F.Cu") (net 4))
 (segment (start 145 91.5) (end 146.2 90.3) (width 0.2) (layer "F.Cu") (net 4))
 (segment (start 141.7425 93.1) (end 142.1 93.1) (width 0.2) (layer "F.Cu") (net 4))
 (segment (start 151.8 91.5) (end 151.3 92) (width 0.2) (layer "F.Cu") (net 4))
 (segment (start 146.2 90.3) (end 148.3 90.3) (width 0.2) (layer "F.Cu") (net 4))
 (segment (start 148.3 90.3) (end 150 92) (width 0.2) (layer "F.Cu") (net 4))
 (segment (start 143.9 91.5) (end 143.8 91.4) (width 0.2) (layer "F.Cu") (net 4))
 (segment (start 143.8 91.4) (end 142.5 90.1) (width 0.2) (layer "F.Cu") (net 4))
 (segment (start 142.1 93.1) (end 143.8 91.4) (width 0.2) (layer "F.Cu") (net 4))
 (segment (start 156.825 91.5) (end 151.8 91.5) (width 0.2) (layer "F.Cu") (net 4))
 (segment (start 150 92) (end 151.3 92) (width 0.2) (layer "F.Cu") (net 4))
 (segment (start 142.5 90.1) (end 141.7425 90.1) (width 0.2) (layer "F.Cu") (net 4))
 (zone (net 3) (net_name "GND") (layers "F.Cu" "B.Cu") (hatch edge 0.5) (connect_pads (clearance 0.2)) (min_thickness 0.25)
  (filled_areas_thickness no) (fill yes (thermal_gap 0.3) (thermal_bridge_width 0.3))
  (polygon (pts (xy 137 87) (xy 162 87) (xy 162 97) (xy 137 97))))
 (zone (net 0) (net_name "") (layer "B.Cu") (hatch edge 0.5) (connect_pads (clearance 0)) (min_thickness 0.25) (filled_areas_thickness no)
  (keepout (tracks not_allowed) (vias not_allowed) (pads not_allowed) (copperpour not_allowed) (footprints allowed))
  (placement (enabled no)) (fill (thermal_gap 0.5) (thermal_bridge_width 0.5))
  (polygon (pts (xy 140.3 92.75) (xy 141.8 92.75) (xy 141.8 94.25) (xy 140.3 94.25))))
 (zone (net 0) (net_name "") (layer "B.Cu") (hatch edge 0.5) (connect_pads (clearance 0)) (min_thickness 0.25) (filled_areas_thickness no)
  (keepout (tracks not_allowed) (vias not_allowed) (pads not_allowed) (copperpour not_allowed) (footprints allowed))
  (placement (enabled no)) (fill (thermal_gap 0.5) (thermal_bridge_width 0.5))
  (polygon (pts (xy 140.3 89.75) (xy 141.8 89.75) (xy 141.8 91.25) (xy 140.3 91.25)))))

